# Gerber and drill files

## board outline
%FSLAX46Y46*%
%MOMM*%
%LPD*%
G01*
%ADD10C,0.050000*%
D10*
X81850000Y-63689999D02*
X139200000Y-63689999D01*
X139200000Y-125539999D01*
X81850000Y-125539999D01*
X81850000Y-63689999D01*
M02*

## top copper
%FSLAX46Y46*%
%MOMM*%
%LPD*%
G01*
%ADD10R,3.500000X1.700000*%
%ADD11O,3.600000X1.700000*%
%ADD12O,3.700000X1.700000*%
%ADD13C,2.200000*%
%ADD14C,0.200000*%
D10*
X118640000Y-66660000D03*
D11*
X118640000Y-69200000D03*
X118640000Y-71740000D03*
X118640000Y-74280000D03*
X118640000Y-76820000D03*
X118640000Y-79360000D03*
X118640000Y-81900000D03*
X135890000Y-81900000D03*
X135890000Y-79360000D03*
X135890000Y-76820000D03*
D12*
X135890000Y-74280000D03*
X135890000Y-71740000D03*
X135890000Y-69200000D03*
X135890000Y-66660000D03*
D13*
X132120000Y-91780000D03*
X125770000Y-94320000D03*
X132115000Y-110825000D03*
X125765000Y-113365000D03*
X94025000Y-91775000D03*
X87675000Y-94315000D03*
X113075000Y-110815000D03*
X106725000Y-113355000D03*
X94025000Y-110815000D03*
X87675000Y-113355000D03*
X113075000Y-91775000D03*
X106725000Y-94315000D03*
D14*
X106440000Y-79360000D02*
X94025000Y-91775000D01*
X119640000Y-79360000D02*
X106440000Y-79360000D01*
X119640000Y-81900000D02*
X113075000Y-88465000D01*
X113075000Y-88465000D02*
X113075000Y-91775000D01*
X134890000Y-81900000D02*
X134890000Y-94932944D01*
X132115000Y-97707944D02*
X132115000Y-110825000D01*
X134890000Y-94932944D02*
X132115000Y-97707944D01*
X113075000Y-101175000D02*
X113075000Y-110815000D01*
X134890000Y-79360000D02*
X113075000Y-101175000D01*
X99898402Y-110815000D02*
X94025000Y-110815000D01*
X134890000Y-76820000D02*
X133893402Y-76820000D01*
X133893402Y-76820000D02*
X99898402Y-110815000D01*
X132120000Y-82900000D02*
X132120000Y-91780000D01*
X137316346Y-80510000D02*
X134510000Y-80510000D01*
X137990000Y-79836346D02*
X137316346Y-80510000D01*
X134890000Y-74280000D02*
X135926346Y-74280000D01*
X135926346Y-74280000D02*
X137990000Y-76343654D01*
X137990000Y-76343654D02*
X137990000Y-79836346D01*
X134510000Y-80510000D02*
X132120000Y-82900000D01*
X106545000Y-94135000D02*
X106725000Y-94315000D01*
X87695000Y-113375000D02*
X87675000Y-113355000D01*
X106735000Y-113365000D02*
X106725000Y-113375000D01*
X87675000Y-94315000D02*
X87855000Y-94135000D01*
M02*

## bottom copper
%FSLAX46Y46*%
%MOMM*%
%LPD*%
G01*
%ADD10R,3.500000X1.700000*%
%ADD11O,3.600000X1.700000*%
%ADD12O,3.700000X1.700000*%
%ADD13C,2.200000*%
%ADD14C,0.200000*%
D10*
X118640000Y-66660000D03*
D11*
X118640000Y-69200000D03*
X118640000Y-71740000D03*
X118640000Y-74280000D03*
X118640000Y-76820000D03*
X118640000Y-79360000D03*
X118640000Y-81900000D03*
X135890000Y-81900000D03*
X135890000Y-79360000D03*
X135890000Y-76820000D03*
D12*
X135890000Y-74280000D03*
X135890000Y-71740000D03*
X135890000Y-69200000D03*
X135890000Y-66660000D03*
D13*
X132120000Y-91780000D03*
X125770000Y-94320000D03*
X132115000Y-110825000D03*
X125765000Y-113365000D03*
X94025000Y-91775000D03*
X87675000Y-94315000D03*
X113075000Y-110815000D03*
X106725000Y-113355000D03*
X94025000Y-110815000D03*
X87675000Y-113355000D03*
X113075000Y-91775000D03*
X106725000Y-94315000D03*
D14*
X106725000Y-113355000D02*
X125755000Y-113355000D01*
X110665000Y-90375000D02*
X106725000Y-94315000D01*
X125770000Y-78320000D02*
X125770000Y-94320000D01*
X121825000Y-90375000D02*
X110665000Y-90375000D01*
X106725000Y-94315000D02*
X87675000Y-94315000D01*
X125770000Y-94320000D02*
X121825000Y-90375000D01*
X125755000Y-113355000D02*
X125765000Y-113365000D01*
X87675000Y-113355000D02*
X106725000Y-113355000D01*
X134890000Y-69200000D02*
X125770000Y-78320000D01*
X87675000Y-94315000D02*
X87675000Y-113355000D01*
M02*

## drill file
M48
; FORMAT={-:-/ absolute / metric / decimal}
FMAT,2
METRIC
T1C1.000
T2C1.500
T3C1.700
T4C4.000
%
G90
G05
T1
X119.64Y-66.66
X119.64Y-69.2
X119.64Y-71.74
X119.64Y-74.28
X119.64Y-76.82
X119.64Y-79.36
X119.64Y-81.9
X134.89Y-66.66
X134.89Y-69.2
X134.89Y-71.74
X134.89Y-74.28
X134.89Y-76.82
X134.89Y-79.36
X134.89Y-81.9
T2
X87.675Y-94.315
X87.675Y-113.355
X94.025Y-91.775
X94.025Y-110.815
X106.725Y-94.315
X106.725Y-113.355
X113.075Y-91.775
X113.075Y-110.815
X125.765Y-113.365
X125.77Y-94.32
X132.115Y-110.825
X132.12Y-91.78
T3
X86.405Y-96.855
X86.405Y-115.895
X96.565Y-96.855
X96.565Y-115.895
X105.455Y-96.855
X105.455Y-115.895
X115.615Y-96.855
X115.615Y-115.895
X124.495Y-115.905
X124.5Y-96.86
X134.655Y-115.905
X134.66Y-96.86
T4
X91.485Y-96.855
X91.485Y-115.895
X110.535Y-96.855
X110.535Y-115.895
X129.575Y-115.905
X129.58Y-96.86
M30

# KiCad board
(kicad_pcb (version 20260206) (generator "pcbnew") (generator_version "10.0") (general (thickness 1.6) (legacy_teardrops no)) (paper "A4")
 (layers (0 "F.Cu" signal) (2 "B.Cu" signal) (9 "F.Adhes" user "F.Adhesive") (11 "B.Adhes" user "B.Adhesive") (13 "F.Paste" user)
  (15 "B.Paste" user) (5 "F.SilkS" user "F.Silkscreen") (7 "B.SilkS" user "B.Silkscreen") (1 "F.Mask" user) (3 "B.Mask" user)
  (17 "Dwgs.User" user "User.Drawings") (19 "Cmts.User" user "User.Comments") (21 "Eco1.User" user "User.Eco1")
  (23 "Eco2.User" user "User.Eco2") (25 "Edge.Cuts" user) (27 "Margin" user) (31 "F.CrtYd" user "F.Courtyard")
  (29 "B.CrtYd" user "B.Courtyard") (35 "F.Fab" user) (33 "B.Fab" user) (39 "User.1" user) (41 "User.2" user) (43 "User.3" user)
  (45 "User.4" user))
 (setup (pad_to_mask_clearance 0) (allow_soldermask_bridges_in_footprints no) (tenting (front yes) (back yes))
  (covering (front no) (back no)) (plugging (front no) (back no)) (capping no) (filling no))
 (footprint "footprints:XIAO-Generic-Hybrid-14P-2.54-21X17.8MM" (layer "F.Cu") (at 127.265 74.28)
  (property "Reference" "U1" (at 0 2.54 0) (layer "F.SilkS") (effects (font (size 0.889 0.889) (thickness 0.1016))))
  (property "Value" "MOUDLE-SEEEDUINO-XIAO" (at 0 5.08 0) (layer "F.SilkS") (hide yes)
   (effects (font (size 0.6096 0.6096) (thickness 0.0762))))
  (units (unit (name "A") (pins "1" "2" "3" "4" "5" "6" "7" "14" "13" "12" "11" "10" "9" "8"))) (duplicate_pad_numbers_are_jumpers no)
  (pad "1" thru_hole rect (at -7.625 -7.62) (size 3.5 1.7) (drill 1 (offset -1 0)) (layers "*.Cu" "*.Mask") (remove_unused_layers no)
   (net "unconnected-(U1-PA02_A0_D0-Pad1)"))
  (pad "2" thru_hole oval (at -7.625 -5.08) (size 3.6 1.7) (drill 1 (offset -1 0)) (layers "*.Cu" "*.Mask") (remove_unused_layers no)
   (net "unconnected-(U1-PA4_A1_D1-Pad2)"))
  (pad "3" thru_hole oval (at -7.625 -2.54) (size 3.6 1.7) (drill 1 (offset -1 0)) (layers "*.Cu" "*.Mask") (remove_unused_layers no)
   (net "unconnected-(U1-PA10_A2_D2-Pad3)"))
  (pad "4" thru_hole oval (at -7.625 0) (size 3.6 1.7) (drill 1 (offset -1 0)) (layers "*.Cu" "*.Mask") (remove_unused_layers no)
   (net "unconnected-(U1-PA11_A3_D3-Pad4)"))
  (pad "5" thru_hole oval (at -7.625 2.54) (size 3.6 1.7) (drill 1 (offset -1 0)) (layers "*.Cu" "*.Mask") (remove_unused_layers no)
   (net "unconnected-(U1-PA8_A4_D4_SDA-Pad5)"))
  (pad "6" thru_hole oval (at -7.625 5.08 180) (size 3.6 1.7) (drill 1 (offset 1 0)) (layers "*.Cu" "*.Mask") (remove_unused_layers no)
   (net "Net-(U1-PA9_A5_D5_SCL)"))
  (pad "7" thru_hole oval (at -7.625 7.62) (size 3.6 1.7) (drill 1 (offset -1 0)) (layers "*.Cu" "*.Mask") (remove_unused_layers no)
   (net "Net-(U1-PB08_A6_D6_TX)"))
  (pad "8" thru_hole oval (at 7.625 7.62) (size 3.6 1.7) (drill 1 (offset 1 0)) (layers "*.Cu" "*.Mask") (remove_unused_layers no)
   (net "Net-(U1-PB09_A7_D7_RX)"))
  (pad "9" thru_hole oval (at 7.625 5.08) (size 3.6 1.7) (drill 1 (offset 1 0)) (layers "*.Cu" "*.Mask") (remove_unused_layers no)
   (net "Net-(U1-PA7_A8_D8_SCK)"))
  (pad "10" thru_hole oval (at 7.625 2.54) (size 3.6 1.7) (drill 1 (offset 1 0)) (layers "*.Cu" "*.Mask") (remove_unused_layers no)
   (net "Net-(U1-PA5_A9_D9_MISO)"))
  (pad "11" thru_hole oval (at 7.625 0) (size 3.7 1.7) (drill 1 (offset 1 0)) (layers "*.Cu" "*.Mask") (remove_unused_layers no)
   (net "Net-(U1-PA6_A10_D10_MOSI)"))
  (pad "12" thru_hole oval (at 7.625 -2.54) (size 3.7 1.7) (drill 1 (offset 1 0)) (layers "*.Cu" "*.Mask") (remove_unused_layers no)
   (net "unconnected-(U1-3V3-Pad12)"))
  (pad "13" thru_hole oval (at 7.625 -5.08) (size 3.7 1.7) (drill 1 (offset 1 0)) (layers "*.Cu" "*.Mask") (remove_unused_layers no)
   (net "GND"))
  (pad "14" thru_hole oval (at 7.625 -7.62) (size 3.7 1.7) (drill 1 (offset 1 0)) (layers "*.Cu" "*.Mask") (remove_unused_layers no)
   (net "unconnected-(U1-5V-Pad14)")))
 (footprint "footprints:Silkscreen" (layer "F.Cu") (at 98.05 72.53)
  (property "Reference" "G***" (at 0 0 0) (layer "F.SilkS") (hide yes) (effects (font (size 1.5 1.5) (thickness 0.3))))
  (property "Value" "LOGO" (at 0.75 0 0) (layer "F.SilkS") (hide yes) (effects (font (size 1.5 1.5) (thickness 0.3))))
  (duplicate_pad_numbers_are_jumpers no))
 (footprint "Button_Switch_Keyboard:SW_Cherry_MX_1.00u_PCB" (layer "F.Cu") (at 132.12 91.78)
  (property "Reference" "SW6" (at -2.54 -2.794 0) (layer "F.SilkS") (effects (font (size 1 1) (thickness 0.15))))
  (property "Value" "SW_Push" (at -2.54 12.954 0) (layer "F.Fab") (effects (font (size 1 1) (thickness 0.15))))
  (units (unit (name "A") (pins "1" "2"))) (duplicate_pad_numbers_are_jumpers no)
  (pad "" np_thru_hole circle (at -7.62 5.08) (size 1.7 1.7) (drill 1.7) (layers "*.Cu" "*.Mask"))
  (pad "" np_thru_hole circle (at -2.54 5.08) (size 4 4) (drill 4) (layers "*.Cu" "*.Mask"))
  (pad "" np_thru_hole circle (at 2.54 5.08) (size 1.7 1.7) (drill 1.7) (layers "*.Cu" "*.Mask"))
  (pad "1" thru_hole circle (at 0 0) (size 2.2 2.2) (drill 1.5) (layers "*.Cu" "*.Mask") (remove_unused_layers no)
   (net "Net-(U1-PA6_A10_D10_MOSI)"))
  (pad "2" thru_hole circle (at -6.35 2.54) (size 2.2 2.2) (drill 1.5) (layers "*.Cu" "*.Mask") (remove_unused_layers no) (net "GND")))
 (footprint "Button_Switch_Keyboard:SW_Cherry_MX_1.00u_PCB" (layer "F.Cu") (at 132.115 110.825)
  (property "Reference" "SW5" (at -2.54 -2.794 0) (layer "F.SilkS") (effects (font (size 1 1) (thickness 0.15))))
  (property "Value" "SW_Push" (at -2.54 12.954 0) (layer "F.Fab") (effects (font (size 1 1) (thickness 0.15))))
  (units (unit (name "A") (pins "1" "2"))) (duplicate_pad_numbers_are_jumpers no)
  (pad "" np_thru_hole circle (at -7.62 5.08) (size 1.7 1.7) (drill 1.7) (layers "*.Cu" "*.Mask"))
  (pad "" np_thru_hole circle (at -2.54 5.08) (size 4 4) (drill 4) (layers "*.Cu" "*.Mask"))
  (pad "" np_thru_hole circle (at 2.54 5.08) (size 1.7 1.7) (drill 1.7) (layers "*.Cu" "*.Mask"))
  (pad "1" thru_hole circle (at 0 0) (size 2.2 2.2) (drill 1.5) (layers "*.Cu" "*.Mask") (remove_unused_layers no)
   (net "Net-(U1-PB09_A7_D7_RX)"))
  (pad "2" thru_hole circle (at -6.35 2.54) (size 2.2 2.2) (drill 1.5) (layers "*.Cu" "*.Mask") (remove_unused_layers no) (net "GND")))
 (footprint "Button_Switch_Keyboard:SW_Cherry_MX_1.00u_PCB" (layer "F.Cu") (at 94.025 91.775)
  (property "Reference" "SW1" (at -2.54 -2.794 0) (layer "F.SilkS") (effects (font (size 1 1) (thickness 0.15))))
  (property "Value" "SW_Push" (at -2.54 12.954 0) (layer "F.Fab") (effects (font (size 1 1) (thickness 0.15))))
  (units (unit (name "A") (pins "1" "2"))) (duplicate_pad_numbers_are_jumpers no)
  (pad "" np_thru_hole circle (at -7.62 5.08) (size 1.7 1.7) (drill 1.7) (layers "*.Cu" "*.Mask"))
  (pad "" np_thru_hole circle (at -2.54 5.08) (size 4 4) (drill 4) (layers "*.Cu" "*.Mask"))
  (pad "" np_thru_hole circle (at 2.54 5.08) (size 1.7 1.7) (drill 1.7) (layers "*.Cu" "*.Mask"))
  (pad "1" thru_hole circle (at 0 0) (size 2.2 2.2) (drill 1.5) (layers "*.Cu" "*.Mask") (remove_unused_layers no)
   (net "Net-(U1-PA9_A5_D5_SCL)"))
  (pad "2" thru_hole circle (at -6.35 2.54) (size 2.2 2.2) (drill 1.5) (layers "*.Cu" "*.Mask") (remove_unused_layers no) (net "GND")))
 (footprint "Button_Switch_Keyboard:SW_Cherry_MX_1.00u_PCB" (layer "F.Cu") (at 113.075 110.815)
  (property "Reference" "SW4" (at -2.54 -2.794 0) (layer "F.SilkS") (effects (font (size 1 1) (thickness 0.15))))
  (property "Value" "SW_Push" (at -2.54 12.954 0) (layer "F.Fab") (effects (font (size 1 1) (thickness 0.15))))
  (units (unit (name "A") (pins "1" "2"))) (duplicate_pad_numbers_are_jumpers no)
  (pad "" np_thru_hole circle (at -7.62 5.08) (size 1.7 1.7) (drill 1.7) (layers "*.Cu" "*.Mask"))
  (pad "" np_thru_hole circle (at -2.54 5.08) (size 4 4) (drill 4) (layers "*.Cu" "*.Mask"))
  (pad "" np_thru_hole circle (at 2.54 5.08) (size 1.7 1.7) (drill 1.7) (layers "*.Cu" "*.Mask"))
  (pad "1" thru_hole circle (at 0 0) (size 2.2 2.2) (drill 1.5) (layers "*.Cu" "*.Mask") (remove_unused_layers no)
   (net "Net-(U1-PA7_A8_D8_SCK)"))
  (pad "2" thru_hole circle (at -6.35 2.54) (size 2.2 2.2) (drill 1.5) (layers "*.Cu" "*.Mask") (remove_unused_layers no) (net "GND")))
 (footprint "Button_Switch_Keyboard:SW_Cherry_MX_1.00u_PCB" (layer "F.Cu") (at 94.025 110.815)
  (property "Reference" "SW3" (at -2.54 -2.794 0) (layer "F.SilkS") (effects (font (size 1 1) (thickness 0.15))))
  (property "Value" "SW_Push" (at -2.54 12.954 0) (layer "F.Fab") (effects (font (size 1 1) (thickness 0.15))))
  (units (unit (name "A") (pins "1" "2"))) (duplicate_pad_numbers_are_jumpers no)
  (pad "" np_thru_hole circle (at -7.62 5.08) (size 1.7 1.7) (drill 1.7) (layers "*.Cu" "*.Mask"))
  (pad "" np_thru_hole circle (at -2.54 5.08) (size 4 4) (drill 4) (layers "*.Cu" "*.Mask"))
  (pad "" np_thru_hole circle (at 2.54 5.08) (size 1.7 1.7) (drill 1.7) (layers "*.Cu" "*.Mask"))
  (pad "1" thru_hole circle (at 0 0) (size 2.2 2.2) (drill 1.5) (layers "*.Cu" "*.Mask") (remove_unused_layers no)
   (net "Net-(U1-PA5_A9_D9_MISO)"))
  (pad "2" thru_hole circle (at -6.35 2.54) (size 2.2 2.2) (drill 1.5) (layers "*.Cu" "*.Mask") (remove_unused_layers no) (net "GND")))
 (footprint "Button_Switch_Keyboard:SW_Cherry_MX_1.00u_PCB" (layer "F.Cu") (at 113.075 91.775)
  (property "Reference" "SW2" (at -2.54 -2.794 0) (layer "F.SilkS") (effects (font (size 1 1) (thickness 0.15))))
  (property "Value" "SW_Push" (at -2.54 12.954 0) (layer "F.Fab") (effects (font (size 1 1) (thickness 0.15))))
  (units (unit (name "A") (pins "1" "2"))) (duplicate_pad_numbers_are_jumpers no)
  (pad "" np_thru_hole circle (at -7.62 5.08) (size 1.7 1.7) (drill 1.7) (layers "*.Cu" "*.Mask"))
  (pad "" np_thru_hole circle (at -2.54 5.08) (size 4 4) (drill 4) (layers "*.Cu" "*.Mask"))
  (pad "" np_thru_hole circle (at 2.54 5.08) (size 1.7 1.7) (drill 1.7) (layers "*.Cu" "*.Mask"))
  (pad "1" thru_hole circle (at 0 0) (size 2.2 2.2) (drill 1.5) (layers "*.Cu" "*.Mask") (remove_unused_layers no)
   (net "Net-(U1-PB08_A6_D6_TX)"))
  (pad "2" thru_hole circle (at -6.35 2.54) (size 2.2 2.2) (drill 1.5) (layers "*.Cu" "*.Mask") (remove_unused_layers no) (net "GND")))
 (gr_rect (start 81.85 63.689999) (end 139.2 125.539999) (stroke (width 0.05) (type default)) (fill no) (layer "Edge.Cuts"))
 (segment (start 106.44 79.36) (end 94.025 91.775) (width 0.2) (layer "F.Cu") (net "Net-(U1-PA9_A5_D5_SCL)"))
 (segment (start 119.64 79.36) (end 106.44 79.36) (width 0.2) (layer "F.Cu") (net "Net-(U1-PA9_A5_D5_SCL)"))
 (segment (start 119.64 81.9) (end 113.075 88.465) (width 0.2) (layer "F.Cu") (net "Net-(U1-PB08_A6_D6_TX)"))
 (segment (start 113.075 88.465) (end 113.075 91.775) (width 0.2) (layer "F.Cu") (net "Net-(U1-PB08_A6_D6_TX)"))
 (segment (start 134.89 81.9) (end 134.89 94.932944) (width 0.2) (layer "F.Cu") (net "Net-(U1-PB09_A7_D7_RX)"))
 (segment (start 132.115 97.707944) (end 132.115 110.825) (width 0.2) (layer "F.Cu") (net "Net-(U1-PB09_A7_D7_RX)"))
 (segment (start 134.89 94.932944) (end 132.115 97.707944) (width 0.2) (layer "F.Cu") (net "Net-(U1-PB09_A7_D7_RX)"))
 (segment (start 113.075 101.175) (end 113.075 110.815) (width 0.2) (layer "F.Cu") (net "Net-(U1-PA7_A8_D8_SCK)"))
 (segment (start 134.89 79.36) (end 113.075 101.175) (width 0.2) (layer "F.Cu") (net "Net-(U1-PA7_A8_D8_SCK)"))
 (segment (start 99.898402 110.815) (end 94.025 110.815) (width 0.2) (layer "F.Cu") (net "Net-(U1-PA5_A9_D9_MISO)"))
 (segment (start 134.89 76.82) (end 133.893402 76.82) (width 0.2) (layer "F.Cu") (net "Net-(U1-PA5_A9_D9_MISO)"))
 (segment (start 133.893402 76.82) (end 99.898402 110.815) (width 0.2) (layer "F.Cu") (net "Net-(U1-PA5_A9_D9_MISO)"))
 (segment (start 132.12 82.9) (end 132.12 91.78) (width 0.2) (layer "F.Cu") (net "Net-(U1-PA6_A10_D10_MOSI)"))
 (segment (start 137.316346 80.51) (end 134.51 80.51) (width 0.2) (layer "F.Cu") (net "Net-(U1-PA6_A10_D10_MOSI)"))
 (segment (start 137.99 79.836346) (end 137.316346 80.51) (width 0.2) (layer "F.Cu") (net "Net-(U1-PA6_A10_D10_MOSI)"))
 (segment (start 134.89 74.28) (end 135.926346 74.28) (width 0.2) (layer "F.Cu") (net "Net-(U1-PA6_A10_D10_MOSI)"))
 (segment (start 135.926346 74.28) (end 137.99 76.343654) (width 0.2) (layer "F.Cu") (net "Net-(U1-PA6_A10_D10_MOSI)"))
 (segment (start 137.99 76.343654) (end 137.99 79.836346) (width 0.2) (layer "F.Cu") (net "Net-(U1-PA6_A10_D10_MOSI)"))
 (segment (start 134.51 80.51) (end 132.12 82.9) (width 0.2) (layer "F.Cu") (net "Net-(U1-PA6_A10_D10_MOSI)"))
 (segment (start 106.545 94.135) (end 106.725 94.315) (width 0.2) (layer "F.Cu") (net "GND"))
 (segment (start 87.695 113.375) (end 87.675 113.355) (width 0.2) (layer "F.Cu") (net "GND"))
 (segment (start 106.735 113.365) (end 106.725 113.375) (width 0.2) (layer "F.Cu") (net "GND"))
 (segment (start 87.675 94.315) (end 87.855 94.135) (width 0.2) (layer "F.Cu") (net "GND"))
 (segment (start 106.725 113.355) (end 125.755 113.355) (width 0.2) (layer "B.Cu") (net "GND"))
 (segment (start 110.665 90.375) (end 106.725 94.315) (width 0.2) (layer "B.Cu") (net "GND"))
 (segment (start 125.77 78.32) (end 125.77 94.32) (width 0.2) (layer "B.Cu") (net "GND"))
 (segment (start 121.825 90.375) (end 110.665 90.375) (width 0.2) (layer "B.Cu") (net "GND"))
 (segment (start 106.725 94.315) (end 87.675 94.315) (width 0.2) (layer "B.Cu") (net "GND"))
 (segment (start 125.77 94.32) (end 121.825 90.375) (width 0.2) (layer "B.Cu") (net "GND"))
 (segment (start 125.755 113.355) (end 125.765 113.365) (width 0.2) (layer "B.Cu") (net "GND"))
 (segment (start 87.675 113.355) (end 106.725 113.355) (width 0.2) (layer "B.Cu") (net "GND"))
 (segment (start 134.89 69.2) (end 125.77 78.32) (width 0.2) (layer "B.Cu") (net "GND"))
 (segment (start 87.675 94.315) (end 87.675 113.355) (width 0.2) (layer "B.Cu") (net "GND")))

